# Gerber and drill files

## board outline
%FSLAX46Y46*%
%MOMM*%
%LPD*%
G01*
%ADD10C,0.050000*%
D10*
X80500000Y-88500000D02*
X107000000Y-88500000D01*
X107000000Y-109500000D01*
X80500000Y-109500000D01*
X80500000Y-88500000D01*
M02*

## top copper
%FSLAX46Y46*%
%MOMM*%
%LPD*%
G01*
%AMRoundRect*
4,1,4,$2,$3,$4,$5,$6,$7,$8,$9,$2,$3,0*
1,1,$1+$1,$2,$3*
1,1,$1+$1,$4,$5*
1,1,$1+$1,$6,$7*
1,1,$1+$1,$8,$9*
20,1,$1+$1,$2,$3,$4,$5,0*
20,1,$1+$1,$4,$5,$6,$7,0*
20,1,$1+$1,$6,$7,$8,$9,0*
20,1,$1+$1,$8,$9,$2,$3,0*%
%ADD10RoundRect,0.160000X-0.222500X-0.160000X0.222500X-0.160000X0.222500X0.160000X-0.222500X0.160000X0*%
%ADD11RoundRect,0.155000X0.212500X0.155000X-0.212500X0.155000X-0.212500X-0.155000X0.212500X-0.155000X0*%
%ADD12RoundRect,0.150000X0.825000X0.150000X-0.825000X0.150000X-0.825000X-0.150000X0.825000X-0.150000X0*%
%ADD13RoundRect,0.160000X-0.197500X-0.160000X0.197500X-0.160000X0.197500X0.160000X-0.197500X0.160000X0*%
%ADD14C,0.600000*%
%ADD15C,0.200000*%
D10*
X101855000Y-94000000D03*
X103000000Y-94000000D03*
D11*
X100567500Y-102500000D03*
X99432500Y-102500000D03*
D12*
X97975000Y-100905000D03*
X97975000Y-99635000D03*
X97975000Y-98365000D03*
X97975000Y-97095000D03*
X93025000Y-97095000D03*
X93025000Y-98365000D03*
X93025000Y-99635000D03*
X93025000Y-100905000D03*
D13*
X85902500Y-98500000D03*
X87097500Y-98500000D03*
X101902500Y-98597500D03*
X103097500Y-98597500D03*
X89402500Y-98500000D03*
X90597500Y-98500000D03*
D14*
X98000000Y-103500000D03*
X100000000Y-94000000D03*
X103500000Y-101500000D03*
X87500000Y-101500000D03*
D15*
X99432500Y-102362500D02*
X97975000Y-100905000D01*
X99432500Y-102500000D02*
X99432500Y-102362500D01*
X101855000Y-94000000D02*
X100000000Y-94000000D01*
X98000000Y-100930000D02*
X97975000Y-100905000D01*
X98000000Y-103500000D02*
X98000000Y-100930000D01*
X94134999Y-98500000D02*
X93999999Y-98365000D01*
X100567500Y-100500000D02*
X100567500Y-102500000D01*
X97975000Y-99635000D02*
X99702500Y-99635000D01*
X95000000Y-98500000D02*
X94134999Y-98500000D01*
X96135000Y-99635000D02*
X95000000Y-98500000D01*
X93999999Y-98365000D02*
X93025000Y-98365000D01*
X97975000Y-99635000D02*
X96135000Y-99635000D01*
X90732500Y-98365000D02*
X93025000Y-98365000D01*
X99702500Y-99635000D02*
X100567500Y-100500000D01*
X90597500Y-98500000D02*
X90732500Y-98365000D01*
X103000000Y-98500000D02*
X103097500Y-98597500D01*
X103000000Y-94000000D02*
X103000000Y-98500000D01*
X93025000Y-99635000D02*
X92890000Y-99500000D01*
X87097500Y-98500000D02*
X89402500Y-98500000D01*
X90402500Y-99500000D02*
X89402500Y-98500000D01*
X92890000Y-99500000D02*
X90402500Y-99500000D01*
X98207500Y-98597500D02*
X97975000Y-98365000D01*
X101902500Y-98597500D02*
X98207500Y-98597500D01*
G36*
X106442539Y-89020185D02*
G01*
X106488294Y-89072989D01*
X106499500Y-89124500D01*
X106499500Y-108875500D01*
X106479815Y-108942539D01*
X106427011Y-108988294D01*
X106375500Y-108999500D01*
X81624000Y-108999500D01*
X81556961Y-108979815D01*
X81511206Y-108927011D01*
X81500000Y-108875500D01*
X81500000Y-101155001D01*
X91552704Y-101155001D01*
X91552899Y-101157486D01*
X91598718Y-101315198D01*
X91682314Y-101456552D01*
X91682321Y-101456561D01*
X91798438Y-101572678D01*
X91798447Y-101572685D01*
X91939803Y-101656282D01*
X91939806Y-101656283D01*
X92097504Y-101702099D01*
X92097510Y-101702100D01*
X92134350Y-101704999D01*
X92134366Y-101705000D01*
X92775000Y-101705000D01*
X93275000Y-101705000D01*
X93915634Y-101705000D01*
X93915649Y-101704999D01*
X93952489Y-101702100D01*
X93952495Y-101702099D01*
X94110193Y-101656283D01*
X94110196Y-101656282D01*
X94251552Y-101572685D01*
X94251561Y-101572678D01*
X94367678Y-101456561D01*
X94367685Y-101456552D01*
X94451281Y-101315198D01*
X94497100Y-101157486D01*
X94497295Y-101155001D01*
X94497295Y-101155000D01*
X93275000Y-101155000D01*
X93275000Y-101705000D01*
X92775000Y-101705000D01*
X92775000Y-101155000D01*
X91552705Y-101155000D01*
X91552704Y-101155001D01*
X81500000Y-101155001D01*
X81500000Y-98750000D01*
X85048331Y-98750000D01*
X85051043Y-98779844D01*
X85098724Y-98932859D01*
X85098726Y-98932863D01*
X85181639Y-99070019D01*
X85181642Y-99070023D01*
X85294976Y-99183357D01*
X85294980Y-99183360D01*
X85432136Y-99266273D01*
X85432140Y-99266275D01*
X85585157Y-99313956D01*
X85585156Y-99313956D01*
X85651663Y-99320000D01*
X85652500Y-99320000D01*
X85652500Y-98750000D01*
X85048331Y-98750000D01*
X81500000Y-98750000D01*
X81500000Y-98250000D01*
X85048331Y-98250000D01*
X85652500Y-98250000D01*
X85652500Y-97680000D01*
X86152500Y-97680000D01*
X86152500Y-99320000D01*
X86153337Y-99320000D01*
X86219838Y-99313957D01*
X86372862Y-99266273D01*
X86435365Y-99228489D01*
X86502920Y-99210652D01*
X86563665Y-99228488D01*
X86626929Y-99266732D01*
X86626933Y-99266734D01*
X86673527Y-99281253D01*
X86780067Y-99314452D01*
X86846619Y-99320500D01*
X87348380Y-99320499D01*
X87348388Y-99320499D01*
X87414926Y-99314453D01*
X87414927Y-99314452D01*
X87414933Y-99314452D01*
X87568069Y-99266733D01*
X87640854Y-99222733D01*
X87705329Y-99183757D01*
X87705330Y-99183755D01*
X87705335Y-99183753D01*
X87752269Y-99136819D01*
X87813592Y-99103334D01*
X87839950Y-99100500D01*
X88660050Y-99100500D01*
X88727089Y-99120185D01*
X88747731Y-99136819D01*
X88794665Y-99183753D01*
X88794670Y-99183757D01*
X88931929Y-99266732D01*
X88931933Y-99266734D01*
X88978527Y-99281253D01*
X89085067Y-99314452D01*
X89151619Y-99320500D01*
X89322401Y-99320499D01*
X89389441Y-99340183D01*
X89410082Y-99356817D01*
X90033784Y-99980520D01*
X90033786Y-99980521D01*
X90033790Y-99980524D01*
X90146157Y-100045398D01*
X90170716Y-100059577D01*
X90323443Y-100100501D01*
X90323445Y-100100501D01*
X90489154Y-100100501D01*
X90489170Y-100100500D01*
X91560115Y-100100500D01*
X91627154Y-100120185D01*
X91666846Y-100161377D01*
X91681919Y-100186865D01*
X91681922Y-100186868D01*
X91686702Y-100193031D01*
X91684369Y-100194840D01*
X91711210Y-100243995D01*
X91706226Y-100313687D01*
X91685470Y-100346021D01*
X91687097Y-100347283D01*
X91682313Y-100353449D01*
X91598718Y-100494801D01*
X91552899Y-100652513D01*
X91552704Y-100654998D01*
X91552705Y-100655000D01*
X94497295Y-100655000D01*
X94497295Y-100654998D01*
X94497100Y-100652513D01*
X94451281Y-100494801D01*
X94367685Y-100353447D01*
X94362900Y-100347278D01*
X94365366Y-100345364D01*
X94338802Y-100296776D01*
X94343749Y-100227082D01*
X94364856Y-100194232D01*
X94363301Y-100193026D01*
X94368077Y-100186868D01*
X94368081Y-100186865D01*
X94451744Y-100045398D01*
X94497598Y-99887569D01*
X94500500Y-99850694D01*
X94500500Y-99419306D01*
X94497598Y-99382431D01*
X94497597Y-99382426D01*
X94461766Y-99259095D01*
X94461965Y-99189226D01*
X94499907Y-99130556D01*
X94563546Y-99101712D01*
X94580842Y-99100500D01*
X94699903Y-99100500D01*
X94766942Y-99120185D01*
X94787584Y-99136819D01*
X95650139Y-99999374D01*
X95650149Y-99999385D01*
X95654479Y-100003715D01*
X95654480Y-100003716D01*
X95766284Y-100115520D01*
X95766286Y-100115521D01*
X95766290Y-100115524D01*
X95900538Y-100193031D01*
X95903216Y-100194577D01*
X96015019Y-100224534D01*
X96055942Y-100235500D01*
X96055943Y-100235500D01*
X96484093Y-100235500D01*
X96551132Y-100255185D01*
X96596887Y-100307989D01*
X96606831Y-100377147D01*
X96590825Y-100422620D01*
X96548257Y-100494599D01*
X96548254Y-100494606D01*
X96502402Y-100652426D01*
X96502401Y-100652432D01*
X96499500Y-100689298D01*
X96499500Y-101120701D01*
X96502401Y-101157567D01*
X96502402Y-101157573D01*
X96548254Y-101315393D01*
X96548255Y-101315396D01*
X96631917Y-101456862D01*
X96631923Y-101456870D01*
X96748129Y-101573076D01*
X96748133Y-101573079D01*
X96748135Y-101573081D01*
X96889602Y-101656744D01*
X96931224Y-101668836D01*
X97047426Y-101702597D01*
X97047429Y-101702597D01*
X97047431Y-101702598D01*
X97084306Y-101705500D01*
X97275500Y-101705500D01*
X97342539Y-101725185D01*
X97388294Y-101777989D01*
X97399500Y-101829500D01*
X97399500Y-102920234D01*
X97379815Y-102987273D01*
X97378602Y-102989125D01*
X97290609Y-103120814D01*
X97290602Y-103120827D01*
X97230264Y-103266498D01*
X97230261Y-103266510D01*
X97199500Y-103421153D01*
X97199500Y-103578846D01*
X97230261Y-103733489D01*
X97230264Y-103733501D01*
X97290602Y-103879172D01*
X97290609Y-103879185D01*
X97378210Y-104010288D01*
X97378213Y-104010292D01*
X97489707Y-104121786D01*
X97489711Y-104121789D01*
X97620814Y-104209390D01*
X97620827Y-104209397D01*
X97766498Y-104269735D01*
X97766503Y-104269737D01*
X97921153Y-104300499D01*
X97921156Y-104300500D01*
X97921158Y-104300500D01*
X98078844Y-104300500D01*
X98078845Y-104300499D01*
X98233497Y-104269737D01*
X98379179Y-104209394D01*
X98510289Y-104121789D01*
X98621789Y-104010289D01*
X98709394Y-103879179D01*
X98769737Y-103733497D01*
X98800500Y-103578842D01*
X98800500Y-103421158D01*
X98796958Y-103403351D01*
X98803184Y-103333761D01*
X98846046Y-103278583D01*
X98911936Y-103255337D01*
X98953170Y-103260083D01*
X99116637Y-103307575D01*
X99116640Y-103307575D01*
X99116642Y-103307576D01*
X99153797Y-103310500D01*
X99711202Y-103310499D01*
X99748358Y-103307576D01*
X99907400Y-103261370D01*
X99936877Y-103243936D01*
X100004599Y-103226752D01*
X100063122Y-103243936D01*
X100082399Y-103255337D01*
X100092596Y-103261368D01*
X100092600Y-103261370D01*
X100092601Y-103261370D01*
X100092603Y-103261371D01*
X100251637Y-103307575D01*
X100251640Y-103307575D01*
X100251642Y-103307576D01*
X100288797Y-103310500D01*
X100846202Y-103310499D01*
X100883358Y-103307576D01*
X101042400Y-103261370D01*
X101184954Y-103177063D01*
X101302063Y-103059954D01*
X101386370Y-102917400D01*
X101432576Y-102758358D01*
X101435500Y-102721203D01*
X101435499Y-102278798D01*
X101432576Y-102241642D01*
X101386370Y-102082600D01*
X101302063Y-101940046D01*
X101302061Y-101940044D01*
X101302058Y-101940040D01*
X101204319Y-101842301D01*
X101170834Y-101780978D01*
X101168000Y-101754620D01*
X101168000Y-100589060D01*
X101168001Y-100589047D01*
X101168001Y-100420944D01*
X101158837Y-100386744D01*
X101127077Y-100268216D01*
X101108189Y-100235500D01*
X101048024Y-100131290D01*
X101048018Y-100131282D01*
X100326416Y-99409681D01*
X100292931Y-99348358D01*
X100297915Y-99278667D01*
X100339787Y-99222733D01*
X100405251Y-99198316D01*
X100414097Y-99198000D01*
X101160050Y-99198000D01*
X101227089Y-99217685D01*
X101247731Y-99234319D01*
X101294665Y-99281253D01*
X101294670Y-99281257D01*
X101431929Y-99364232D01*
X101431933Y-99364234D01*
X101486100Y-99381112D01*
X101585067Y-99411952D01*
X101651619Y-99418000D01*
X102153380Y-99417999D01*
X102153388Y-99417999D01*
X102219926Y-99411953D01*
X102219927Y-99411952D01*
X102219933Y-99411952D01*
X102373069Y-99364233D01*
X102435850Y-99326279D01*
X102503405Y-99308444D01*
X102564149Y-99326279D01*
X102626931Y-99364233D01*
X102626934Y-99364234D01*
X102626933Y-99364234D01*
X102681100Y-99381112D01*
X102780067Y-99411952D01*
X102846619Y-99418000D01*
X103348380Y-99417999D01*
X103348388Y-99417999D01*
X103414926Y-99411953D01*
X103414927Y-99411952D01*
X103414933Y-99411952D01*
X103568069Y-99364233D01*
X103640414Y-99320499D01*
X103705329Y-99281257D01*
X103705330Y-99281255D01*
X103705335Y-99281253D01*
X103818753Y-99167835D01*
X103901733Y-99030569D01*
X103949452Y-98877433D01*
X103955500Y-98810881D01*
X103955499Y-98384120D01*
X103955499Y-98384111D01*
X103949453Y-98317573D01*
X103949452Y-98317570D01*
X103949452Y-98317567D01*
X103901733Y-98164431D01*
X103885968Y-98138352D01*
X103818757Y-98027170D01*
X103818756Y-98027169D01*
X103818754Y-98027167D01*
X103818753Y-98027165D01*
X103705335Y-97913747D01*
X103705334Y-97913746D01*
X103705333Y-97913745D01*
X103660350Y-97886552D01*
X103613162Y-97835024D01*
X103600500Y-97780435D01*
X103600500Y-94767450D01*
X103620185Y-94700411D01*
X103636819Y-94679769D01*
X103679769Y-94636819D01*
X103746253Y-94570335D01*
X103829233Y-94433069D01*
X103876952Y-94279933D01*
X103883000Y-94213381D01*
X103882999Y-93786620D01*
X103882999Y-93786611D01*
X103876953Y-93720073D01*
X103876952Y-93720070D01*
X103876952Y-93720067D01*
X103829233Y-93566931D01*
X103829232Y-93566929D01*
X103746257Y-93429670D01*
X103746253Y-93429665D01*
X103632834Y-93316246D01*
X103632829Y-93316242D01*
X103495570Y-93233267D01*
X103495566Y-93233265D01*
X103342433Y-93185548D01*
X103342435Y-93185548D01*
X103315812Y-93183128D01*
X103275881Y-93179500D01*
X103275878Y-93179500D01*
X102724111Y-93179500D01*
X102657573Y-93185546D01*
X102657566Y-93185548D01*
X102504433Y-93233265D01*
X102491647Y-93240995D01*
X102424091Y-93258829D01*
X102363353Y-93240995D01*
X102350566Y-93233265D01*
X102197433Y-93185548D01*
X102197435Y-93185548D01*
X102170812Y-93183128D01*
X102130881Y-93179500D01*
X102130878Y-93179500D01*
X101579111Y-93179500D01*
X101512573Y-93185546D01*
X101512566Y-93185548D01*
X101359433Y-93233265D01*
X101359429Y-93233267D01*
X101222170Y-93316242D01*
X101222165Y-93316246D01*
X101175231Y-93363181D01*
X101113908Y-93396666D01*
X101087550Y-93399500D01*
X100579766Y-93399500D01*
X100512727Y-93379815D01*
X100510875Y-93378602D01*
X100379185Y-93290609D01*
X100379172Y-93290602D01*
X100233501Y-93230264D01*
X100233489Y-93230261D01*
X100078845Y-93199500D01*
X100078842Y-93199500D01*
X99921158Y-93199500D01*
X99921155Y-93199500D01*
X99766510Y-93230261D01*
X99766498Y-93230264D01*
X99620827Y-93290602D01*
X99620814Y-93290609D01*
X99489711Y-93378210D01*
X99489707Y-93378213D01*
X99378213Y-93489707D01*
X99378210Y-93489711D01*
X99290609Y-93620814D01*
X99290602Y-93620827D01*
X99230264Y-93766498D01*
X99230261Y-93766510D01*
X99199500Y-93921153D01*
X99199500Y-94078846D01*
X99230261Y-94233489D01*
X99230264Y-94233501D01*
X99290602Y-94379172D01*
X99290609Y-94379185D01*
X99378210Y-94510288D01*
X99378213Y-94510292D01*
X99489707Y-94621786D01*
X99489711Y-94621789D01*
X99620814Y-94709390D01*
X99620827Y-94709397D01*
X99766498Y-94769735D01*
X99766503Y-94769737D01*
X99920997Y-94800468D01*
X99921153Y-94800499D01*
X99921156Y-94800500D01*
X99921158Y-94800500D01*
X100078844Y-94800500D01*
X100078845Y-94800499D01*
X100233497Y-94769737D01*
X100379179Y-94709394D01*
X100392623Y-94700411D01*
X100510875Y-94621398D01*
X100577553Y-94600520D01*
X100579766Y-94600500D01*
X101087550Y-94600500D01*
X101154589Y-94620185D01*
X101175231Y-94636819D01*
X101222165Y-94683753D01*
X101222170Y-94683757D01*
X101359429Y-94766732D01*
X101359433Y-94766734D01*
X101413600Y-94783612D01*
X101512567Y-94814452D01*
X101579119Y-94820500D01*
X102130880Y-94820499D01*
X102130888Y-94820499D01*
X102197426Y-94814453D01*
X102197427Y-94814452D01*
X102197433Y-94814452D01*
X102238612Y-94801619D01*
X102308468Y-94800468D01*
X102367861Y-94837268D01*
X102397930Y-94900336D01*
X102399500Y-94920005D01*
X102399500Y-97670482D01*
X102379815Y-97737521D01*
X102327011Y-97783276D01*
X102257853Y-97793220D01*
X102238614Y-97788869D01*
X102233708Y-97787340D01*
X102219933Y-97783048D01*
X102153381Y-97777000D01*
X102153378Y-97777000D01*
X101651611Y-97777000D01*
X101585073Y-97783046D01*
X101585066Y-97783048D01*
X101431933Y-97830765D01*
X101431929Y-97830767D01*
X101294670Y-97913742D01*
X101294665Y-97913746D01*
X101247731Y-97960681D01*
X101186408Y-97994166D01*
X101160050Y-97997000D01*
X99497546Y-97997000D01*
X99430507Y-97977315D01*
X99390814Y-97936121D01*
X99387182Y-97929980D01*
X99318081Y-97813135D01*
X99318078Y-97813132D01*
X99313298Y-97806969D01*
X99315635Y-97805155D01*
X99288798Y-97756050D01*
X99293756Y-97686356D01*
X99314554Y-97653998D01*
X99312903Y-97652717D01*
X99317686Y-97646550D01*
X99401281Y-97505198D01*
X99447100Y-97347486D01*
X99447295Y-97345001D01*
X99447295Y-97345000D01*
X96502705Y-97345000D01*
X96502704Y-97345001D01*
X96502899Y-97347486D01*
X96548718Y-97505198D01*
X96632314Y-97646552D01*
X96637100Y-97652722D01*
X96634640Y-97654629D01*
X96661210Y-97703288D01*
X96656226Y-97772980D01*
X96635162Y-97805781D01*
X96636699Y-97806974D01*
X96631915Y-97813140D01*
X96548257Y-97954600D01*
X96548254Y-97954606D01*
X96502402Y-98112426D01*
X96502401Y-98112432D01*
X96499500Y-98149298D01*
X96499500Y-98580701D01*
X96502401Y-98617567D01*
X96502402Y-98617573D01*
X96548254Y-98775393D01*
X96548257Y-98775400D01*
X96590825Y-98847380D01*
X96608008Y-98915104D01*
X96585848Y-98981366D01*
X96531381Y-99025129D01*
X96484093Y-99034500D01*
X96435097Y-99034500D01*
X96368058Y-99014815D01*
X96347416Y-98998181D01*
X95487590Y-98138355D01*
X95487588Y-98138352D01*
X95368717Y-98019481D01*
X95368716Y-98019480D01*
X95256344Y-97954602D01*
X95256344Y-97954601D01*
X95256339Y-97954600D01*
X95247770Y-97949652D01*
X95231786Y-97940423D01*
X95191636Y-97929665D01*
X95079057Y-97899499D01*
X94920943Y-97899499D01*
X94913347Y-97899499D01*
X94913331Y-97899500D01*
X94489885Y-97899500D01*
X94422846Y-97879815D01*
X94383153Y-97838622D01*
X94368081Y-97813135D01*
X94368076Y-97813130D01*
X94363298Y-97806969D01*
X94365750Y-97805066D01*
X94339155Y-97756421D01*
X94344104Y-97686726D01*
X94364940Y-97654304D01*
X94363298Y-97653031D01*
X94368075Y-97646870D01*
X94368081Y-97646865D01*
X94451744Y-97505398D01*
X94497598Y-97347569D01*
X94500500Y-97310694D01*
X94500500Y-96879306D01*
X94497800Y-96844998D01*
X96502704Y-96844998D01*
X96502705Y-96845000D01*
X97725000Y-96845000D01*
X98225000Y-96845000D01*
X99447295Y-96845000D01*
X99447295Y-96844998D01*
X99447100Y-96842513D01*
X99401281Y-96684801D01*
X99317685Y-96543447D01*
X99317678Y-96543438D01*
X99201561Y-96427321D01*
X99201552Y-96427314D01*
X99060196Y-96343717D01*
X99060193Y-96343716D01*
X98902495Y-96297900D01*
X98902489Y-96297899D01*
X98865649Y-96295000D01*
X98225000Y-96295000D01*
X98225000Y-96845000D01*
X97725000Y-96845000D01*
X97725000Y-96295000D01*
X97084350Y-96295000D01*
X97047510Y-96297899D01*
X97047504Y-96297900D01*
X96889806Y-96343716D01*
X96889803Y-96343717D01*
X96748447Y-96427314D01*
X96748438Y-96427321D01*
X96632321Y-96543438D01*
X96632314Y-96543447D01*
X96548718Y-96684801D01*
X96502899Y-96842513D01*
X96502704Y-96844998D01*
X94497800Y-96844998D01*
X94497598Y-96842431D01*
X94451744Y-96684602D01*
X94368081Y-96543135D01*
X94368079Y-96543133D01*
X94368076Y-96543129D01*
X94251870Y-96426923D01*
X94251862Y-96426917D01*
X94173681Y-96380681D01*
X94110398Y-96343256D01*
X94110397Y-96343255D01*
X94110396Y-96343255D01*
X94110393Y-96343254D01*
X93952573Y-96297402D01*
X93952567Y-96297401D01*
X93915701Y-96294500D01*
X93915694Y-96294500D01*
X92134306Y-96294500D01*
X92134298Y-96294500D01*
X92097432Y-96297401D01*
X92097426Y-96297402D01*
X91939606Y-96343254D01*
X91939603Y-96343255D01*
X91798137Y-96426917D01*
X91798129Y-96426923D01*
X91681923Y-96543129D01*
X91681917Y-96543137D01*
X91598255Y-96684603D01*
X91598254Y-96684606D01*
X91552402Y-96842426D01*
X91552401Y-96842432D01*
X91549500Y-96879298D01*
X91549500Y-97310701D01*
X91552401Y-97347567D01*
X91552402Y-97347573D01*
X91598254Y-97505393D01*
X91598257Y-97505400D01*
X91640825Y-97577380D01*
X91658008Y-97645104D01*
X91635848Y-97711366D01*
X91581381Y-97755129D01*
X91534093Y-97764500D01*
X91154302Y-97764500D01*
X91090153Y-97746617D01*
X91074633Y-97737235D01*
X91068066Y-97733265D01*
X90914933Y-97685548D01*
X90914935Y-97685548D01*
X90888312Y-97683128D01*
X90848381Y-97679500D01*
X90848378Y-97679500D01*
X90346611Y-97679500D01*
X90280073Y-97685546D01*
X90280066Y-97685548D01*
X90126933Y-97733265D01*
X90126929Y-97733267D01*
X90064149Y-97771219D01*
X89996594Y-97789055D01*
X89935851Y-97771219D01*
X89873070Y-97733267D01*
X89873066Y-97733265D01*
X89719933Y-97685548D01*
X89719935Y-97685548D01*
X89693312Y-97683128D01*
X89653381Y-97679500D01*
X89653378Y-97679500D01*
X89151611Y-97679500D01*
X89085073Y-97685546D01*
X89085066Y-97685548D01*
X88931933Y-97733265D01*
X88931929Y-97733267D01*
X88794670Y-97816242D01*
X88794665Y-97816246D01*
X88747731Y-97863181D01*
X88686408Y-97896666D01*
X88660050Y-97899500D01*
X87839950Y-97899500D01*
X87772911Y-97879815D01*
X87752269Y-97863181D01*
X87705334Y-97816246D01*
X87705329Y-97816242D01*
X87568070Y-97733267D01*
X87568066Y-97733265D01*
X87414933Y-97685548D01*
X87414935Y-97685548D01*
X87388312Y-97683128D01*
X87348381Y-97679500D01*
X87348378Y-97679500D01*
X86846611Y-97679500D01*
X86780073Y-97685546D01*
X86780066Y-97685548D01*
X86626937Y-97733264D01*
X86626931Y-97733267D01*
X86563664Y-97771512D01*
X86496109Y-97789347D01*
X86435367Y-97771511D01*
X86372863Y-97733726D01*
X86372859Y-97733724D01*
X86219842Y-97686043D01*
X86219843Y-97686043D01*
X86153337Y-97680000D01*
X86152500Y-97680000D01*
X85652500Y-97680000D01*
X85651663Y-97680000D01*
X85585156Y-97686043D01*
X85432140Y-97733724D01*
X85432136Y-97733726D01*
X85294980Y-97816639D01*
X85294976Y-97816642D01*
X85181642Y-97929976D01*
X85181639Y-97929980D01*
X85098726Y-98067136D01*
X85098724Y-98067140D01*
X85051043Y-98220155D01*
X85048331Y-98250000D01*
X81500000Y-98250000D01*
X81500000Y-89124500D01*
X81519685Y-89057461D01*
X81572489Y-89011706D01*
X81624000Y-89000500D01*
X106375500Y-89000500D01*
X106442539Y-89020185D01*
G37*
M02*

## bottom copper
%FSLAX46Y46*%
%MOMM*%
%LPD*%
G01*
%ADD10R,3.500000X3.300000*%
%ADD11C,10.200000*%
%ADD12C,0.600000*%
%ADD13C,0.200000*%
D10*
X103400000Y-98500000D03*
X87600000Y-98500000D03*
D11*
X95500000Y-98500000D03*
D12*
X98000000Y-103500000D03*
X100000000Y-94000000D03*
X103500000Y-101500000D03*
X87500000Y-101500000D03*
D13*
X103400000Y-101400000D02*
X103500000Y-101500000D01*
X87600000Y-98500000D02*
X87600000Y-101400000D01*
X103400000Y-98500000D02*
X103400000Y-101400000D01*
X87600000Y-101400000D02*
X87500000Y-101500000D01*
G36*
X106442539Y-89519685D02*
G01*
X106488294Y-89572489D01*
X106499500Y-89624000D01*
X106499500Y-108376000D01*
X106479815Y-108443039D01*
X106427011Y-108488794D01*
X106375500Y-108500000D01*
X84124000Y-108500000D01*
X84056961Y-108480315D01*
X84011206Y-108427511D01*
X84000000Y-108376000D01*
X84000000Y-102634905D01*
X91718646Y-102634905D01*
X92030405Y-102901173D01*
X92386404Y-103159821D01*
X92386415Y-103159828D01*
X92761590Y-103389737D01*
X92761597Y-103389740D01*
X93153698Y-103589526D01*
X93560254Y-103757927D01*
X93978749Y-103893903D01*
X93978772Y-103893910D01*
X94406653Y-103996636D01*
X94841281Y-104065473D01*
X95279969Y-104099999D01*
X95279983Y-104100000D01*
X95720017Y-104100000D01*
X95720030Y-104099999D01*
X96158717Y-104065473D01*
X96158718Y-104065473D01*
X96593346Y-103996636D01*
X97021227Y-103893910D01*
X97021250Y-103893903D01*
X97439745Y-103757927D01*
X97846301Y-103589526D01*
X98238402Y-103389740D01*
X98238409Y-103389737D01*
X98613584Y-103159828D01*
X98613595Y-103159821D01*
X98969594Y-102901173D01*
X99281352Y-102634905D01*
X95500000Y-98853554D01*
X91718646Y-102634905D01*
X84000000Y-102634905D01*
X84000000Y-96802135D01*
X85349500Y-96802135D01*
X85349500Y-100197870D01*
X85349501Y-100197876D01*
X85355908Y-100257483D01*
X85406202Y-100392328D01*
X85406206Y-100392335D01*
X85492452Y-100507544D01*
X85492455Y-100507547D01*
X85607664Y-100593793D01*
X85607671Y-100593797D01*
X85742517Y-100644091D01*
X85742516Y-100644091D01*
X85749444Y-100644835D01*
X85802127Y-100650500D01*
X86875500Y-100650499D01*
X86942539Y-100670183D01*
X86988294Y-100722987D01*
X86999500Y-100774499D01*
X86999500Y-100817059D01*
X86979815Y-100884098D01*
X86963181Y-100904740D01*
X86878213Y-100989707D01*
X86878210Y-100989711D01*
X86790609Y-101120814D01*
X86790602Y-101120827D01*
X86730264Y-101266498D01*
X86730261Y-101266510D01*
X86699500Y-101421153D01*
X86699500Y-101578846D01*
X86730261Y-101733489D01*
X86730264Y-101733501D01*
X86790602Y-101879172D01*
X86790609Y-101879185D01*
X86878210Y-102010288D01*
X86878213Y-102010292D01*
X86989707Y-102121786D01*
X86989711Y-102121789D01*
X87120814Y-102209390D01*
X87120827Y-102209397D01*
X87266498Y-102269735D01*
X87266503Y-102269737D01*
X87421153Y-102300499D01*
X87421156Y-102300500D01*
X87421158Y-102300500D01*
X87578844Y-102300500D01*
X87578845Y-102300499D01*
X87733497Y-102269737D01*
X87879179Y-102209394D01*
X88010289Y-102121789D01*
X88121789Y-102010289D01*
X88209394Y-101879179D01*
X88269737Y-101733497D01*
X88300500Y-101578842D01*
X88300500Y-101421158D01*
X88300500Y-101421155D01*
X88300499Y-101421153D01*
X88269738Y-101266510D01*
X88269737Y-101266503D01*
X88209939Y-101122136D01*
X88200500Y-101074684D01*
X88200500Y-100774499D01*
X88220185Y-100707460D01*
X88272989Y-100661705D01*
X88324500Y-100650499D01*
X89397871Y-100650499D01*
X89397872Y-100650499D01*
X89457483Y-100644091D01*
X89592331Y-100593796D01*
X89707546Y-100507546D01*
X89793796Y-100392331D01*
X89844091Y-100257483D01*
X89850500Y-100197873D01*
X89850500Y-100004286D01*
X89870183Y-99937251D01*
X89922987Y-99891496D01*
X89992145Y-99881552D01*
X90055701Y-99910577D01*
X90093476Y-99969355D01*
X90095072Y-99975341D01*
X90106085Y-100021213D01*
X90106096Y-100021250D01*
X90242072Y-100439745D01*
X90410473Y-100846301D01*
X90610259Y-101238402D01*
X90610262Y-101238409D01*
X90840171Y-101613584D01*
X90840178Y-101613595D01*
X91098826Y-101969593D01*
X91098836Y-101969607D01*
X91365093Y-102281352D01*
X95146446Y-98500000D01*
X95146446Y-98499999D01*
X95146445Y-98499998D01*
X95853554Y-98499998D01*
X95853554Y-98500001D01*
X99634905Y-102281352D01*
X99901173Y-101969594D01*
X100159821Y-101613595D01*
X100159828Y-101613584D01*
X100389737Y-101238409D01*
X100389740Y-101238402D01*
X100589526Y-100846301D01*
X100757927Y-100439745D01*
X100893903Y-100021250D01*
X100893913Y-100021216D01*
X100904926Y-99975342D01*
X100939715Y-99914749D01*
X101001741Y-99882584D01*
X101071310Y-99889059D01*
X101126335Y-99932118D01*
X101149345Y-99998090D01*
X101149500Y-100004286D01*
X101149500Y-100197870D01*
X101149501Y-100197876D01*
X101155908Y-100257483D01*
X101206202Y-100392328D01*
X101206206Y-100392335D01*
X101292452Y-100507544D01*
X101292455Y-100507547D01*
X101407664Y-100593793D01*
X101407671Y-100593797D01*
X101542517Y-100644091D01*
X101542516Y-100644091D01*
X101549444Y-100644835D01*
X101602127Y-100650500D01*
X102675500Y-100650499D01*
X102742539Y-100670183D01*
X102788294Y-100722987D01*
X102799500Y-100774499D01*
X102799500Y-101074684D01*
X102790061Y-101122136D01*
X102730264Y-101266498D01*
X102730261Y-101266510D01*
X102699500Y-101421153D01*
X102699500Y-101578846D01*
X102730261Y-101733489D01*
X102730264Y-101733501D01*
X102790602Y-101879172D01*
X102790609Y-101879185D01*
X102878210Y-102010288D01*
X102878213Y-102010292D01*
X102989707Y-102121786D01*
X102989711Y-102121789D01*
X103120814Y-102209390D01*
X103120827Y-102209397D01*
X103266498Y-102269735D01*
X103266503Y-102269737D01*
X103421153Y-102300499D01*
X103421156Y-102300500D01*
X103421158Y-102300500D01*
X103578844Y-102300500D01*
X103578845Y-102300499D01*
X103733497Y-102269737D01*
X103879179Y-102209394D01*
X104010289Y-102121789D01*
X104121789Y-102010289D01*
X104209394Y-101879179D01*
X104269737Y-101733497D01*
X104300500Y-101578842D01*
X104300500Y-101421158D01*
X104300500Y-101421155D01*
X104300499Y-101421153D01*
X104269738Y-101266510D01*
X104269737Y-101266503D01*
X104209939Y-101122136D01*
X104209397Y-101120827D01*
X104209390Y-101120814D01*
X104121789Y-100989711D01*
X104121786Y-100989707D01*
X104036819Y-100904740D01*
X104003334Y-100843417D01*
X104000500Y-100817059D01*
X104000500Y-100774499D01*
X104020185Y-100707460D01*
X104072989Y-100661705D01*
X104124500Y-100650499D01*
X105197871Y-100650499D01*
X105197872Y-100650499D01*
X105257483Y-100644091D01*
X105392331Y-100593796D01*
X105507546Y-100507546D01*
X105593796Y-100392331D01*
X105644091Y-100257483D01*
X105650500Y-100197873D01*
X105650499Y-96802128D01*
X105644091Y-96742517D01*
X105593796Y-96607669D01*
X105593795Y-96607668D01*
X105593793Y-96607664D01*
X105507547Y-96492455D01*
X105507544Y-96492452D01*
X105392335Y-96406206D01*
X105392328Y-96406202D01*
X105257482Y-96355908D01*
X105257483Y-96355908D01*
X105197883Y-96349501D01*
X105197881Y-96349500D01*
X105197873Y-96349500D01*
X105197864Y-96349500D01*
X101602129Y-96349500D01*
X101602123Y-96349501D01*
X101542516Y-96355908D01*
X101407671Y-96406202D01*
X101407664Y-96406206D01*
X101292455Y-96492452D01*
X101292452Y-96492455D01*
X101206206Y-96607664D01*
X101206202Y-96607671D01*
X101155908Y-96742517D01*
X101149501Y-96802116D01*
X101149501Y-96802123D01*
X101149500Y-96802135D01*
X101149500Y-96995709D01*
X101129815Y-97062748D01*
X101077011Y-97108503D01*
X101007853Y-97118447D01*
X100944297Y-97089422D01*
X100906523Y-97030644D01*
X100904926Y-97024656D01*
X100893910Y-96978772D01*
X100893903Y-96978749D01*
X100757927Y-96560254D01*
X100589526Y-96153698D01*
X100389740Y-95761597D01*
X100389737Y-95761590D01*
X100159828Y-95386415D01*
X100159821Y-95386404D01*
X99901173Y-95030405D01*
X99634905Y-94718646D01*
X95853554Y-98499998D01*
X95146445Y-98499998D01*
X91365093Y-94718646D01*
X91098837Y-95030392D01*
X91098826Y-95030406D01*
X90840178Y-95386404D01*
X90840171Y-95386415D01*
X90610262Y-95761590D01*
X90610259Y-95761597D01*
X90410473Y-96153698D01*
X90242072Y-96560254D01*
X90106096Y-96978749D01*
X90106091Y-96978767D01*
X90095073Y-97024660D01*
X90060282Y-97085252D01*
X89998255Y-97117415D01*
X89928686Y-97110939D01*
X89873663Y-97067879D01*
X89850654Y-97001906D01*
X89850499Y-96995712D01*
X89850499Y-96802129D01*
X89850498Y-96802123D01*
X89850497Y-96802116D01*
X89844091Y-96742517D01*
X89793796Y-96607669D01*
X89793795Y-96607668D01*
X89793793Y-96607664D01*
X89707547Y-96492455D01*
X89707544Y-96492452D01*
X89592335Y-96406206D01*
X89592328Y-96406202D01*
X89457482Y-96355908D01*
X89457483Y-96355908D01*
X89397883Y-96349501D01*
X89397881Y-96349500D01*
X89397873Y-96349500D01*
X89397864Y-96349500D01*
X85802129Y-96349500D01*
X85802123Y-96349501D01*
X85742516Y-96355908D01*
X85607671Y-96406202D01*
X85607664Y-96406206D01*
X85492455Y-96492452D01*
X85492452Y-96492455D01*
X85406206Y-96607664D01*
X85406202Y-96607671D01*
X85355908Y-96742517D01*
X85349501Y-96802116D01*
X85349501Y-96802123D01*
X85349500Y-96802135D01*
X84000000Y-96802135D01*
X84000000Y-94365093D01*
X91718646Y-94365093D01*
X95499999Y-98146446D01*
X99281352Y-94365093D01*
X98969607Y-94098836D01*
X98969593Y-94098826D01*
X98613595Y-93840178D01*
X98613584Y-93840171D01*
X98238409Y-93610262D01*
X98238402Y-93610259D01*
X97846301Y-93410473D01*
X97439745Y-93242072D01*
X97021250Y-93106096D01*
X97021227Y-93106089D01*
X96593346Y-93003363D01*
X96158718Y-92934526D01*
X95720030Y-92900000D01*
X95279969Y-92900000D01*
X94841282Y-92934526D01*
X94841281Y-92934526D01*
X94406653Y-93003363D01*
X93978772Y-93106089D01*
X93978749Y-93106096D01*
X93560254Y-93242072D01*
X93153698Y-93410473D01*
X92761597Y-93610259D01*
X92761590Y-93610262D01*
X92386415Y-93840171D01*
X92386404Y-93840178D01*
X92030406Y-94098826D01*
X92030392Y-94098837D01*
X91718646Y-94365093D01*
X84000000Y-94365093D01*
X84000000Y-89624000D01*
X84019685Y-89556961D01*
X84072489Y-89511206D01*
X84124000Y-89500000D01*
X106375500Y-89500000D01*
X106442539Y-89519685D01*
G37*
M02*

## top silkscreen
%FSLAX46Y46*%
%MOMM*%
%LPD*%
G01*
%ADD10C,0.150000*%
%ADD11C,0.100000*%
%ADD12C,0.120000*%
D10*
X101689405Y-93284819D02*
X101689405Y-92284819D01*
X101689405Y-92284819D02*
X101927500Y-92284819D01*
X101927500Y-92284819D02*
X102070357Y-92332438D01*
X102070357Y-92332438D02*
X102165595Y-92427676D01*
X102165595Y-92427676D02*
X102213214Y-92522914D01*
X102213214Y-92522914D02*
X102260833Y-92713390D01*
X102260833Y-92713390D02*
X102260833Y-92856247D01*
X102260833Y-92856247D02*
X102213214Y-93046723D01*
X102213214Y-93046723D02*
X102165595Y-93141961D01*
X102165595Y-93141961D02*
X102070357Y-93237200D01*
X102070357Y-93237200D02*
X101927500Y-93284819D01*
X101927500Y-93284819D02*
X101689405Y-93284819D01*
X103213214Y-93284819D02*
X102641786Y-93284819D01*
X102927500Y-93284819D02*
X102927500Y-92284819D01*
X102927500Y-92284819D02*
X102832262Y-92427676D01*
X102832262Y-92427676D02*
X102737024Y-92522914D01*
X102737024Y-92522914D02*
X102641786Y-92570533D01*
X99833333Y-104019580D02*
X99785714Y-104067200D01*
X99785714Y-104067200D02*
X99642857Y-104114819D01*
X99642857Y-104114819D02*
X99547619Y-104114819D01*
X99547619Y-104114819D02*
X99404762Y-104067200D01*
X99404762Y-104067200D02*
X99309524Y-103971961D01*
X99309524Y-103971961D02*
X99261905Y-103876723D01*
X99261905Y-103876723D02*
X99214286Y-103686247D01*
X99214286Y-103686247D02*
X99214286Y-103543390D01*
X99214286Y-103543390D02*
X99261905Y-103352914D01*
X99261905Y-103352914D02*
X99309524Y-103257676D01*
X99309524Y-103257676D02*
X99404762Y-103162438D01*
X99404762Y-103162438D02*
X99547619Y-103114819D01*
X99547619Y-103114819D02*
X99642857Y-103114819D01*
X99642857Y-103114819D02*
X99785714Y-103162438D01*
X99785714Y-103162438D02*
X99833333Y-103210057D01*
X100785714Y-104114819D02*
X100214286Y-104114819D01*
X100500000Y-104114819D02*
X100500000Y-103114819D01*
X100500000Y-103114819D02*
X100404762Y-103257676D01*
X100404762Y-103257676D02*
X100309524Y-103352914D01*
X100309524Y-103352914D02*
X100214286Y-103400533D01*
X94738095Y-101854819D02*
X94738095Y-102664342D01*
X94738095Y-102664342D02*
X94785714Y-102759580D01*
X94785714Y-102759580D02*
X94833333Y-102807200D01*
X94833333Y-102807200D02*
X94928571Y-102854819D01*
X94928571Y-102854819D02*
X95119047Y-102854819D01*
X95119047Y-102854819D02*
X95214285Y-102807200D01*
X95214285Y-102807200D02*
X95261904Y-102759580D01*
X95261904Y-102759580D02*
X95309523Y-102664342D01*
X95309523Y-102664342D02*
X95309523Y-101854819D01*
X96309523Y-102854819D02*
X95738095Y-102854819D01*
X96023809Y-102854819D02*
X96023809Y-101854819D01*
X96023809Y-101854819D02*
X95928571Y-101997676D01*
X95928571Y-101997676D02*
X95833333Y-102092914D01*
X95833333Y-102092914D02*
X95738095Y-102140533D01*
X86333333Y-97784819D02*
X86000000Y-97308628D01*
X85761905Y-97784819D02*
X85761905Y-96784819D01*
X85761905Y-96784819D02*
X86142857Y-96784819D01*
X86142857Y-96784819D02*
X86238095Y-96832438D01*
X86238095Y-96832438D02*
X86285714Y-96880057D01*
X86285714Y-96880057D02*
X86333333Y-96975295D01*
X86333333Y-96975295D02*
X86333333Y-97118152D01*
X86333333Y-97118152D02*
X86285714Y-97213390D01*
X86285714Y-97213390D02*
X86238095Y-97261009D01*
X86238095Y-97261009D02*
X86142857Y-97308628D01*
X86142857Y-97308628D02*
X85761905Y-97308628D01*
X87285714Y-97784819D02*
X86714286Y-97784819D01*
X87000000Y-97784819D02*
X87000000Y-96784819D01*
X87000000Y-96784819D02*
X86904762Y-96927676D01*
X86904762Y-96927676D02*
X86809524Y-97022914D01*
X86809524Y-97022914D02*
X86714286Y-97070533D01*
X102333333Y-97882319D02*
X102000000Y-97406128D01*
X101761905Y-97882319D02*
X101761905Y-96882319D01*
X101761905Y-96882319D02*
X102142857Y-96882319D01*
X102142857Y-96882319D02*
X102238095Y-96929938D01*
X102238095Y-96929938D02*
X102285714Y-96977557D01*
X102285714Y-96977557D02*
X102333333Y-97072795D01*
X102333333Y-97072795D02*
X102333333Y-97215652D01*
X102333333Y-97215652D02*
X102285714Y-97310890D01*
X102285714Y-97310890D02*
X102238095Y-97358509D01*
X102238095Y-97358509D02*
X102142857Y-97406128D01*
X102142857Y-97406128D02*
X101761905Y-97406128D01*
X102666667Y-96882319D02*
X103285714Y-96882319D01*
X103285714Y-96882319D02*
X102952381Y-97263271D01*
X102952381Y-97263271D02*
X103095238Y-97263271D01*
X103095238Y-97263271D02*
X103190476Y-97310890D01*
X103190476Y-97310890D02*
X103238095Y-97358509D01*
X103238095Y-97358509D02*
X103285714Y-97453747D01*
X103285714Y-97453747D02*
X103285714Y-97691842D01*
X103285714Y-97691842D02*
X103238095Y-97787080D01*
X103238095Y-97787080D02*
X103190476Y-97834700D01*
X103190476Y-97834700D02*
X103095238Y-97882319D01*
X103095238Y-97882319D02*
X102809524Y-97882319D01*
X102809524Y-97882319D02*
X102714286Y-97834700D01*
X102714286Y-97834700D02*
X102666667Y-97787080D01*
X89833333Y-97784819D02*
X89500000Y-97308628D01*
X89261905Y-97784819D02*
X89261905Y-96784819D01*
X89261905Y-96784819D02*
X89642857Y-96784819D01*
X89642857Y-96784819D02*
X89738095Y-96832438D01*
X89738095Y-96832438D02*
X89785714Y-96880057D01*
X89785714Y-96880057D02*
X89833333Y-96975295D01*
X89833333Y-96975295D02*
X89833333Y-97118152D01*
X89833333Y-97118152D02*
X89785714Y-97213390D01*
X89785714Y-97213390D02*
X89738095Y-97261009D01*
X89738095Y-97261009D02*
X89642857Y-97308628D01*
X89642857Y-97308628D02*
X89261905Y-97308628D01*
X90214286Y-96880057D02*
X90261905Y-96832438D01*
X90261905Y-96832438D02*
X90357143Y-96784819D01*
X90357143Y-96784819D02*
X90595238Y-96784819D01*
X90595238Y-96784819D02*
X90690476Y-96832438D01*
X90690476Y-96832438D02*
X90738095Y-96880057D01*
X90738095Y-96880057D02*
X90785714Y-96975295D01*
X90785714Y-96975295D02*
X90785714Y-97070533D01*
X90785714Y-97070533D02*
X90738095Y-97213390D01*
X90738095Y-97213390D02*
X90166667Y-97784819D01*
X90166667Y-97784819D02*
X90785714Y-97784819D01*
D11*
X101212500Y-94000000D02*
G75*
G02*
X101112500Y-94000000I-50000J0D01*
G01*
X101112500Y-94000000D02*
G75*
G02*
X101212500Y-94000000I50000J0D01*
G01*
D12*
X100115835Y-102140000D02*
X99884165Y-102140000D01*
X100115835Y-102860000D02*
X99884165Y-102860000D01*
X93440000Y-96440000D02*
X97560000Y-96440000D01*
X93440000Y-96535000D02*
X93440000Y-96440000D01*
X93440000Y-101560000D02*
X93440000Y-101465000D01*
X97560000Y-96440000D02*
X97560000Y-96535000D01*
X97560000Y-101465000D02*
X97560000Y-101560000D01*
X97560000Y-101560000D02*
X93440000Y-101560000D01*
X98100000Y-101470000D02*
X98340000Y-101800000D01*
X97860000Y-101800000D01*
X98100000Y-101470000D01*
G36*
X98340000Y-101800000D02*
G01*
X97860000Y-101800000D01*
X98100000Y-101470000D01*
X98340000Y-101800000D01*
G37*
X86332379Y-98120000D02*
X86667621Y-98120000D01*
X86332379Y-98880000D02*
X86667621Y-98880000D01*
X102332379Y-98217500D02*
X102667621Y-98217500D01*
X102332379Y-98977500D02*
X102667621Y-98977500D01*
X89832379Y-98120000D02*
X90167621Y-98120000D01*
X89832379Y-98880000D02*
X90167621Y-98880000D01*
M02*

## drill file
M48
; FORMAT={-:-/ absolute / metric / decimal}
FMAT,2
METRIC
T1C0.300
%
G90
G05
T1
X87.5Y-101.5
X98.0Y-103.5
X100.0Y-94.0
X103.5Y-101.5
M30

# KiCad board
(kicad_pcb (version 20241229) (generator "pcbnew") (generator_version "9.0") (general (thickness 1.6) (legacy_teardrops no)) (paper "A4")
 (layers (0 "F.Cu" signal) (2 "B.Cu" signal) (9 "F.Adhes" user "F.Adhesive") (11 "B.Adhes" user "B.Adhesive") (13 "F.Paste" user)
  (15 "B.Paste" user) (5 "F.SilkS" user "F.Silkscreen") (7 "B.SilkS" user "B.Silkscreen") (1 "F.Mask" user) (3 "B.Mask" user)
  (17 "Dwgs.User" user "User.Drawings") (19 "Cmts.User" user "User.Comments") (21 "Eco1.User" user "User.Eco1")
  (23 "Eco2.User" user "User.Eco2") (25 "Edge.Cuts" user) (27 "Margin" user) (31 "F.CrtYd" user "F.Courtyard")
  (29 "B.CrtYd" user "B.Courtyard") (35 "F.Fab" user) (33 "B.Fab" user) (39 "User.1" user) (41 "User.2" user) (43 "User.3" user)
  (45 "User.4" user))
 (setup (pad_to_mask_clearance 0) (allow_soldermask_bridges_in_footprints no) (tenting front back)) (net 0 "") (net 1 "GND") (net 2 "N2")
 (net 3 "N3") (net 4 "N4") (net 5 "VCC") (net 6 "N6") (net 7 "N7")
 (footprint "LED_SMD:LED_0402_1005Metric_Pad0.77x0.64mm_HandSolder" (layer "F.Cu") (at 102.4275 94)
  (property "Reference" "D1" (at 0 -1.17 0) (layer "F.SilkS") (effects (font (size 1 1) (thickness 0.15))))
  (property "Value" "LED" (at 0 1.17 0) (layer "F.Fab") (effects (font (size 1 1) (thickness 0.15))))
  (fp_circle (center -1.265 0) (end -1.215 0) (stroke (width 0.1) (type solid)) (fill no) (layer "F.SilkS"))
  (pad "1" smd roundrect (at -0.5725 0) (size 0.765 0.64) (layers "F.Cu" "F.Mask" "F.Paste") (roundrect_rratio 0.25) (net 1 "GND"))
  (pad "2" smd roundrect (at 0.5725 0) (size 0.765 0.64) (layers "F.Cu" "F.Mask" "F.Paste") (roundrect_rratio 0.25) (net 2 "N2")))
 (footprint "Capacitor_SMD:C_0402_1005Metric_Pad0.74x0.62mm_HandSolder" (layer "F.Cu") (at 100 102.5 180)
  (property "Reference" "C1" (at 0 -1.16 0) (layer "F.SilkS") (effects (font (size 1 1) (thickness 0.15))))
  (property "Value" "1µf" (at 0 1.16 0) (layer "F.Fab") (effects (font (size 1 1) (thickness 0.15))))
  (fp_line (start -0.115835 0.36) (end 0.115835 0.36) (stroke (width 0.12) (type solid)) (layer "F.SilkS"))
  (fp_line (start -0.115835 -0.36) (end 0.115835 -0.36) (stroke (width 0.12) (type solid)) (layer "F.SilkS"))
  (pad "1" smd roundrect (at -0.5675 0 180) (size 0.735 0.62) (layers "F.Cu" "F.Mask" "F.Paste") (roundrect_rratio 0.25) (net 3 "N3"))
  (pad "2" smd roundrect (at 0.5675 0 180) (size 0.735 0.62) (layers "F.Cu" "F.Mask" "F.Paste") (roundrect_rratio 0.25) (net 1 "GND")))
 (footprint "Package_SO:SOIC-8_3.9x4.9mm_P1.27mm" (layer "F.Cu") (at 95.5 99 180)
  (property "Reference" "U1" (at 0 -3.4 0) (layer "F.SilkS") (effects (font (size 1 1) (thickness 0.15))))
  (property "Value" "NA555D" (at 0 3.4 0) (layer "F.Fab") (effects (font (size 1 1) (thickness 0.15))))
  (fp_line (start 2.06 2.56) (end -2.06 2.56) (stroke (width 0.12) (type solid)) (layer "F.SilkS"))
  (fp_line (start 2.06 2.465) (end 2.06 2.56) (stroke (width 0.12) (type solid)) (layer "F.SilkS"))
  (fp_line (start 2.06 -2.56) (end 2.06 -2.465) (stroke (width 0.12) (type solid)) (layer "F.SilkS"))
  (fp_line (start -2.06 2.56) (end -2.06 2.465) (stroke (width 0.12) (type solid)) (layer "F.SilkS"))
  (fp_line (start -2.06 -2.465) (end -2.06 -2.56) (stroke (width 0.12) (type solid)) (layer "F.SilkS"))
  (fp_line (start -2.06 -2.56) (end 2.06 -2.56) (stroke (width 0.12) (type solid)) (layer "F.SilkS"))
  (fp_poly (pts (xy -2.6 -2.47) (xy -2.84 -2.8) (xy -2.36 -2.8)) (stroke (width 0.12) (type solid)) (fill yes) (layer "F.SilkS"))
  (pad "1" smd roundrect (at -2.475 -1.905 180) (size 1.95 0.6) (layers "F.Cu" "F.Mask" "F.Paste") (roundrect_rratio 0.25) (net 1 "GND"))
  (pad "2" smd roundrect (at -2.475 -0.635 180) (size 1.95 0.6) (layers "F.Cu" "F.Mask" "F.Paste") (roundrect_rratio 0.25) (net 3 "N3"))
  (pad "3" smd roundrect (at -2.475 0.635 180) (size 1.95 0.6) (layers "F.Cu" "F.Mask" "F.Paste") (roundrect_rratio 0.25) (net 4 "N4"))
  (pad "4" smd roundrect (at -2.475 1.905 180) (size 1.95 0.6) (layers "F.Cu" "F.Mask" "F.Paste") (roundrect_rratio 0.25) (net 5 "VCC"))
  (pad "5" smd roundrect (at 2.475 1.905 180) (size 1.95 0.6) (layers "F.Cu" "F.Mask" "F.Paste") (roundrect_rratio 0.25) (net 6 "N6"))
  (pad "6" smd roundrect (at 2.475 0.635 180) (size 1.95 0.6) (layers "F.Cu" "F.Mask" "F.Paste") (roundrect_rratio 0.25) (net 3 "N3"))
  (pad "7" smd roundrect (at 2.475 -0.635 180) (size 1.95 0.6) (layers "F.Cu" "F.Mask" "F.Paste") (roundrect_rratio 0.25) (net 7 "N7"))
  (pad "8" smd roundrect (at 2.475 -1.905 180) (size 1.95 0.6) (layers "F.Cu" "F.Mask" "F.Paste") (roundrect_rratio 0.25) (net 5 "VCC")))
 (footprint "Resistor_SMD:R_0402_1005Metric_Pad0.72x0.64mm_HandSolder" (layer "F.Cu") (at 86.5 98.5)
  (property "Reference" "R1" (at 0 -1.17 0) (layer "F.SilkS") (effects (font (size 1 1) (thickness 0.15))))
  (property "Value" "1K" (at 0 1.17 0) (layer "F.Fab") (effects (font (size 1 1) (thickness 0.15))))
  (fp_line (start -0.167621 -0.38) (end 0.167621 -0.38) (stroke (width 0.12) (type solid)) (layer "F.SilkS"))
  (fp_line (start -0.167621 0.38) (end 0.167621 0.38) (stroke (width 0.12) (type solid)) (layer "F.SilkS"))
  (pad "1" smd roundrect (at -0.5975 0) (size 0.715 0.64) (layers "F.Cu" "F.Mask" "F.Paste") (roundrect_rratio 0.25) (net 5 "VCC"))
  (pad "2" smd roundrect (at 0.5975 0) (size 0.715 0.64) (layers "F.Cu" "F.Mask" "F.Paste") (roundrect_rratio 0.25) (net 7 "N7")))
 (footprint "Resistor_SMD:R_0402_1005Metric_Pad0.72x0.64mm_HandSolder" (layer "F.Cu") (at 102.5 98.5975)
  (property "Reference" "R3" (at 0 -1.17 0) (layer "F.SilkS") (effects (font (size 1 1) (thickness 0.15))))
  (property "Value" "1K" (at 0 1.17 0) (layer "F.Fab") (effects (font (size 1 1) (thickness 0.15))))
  (fp_line (start -0.167621 -0.38) (end 0.167621 -0.38) (stroke (width 0.12) (type solid)) (layer "F.SilkS"))
  (fp_line (start -0.167621 0.38) (end 0.167621 0.38) (stroke (width 0.12) (type solid)) (layer "F.SilkS"))
  (pad "1" smd roundrect (at -0.5975 0) (size 0.715 0.64) (layers "F.Cu" "F.Mask" "F.Paste") (roundrect_rratio 0.25) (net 4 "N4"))
  (pad "2" smd roundrect (at 0.5975 0) (size 0.715 0.64) (layers "F.Cu" "F.Mask" "F.Paste") (roundrect_rratio 0.25) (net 2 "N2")))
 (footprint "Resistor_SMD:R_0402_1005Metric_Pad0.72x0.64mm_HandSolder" (layer "F.Cu") (at 90 98.5)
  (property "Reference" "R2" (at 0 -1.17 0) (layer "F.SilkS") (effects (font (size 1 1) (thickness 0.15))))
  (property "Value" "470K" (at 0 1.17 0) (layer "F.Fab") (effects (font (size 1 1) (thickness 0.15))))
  (fp_line (start -0.167621 -0.38) (end 0.167621 -0.38) (stroke (width 0.12) (type solid)) (layer "F.SilkS"))
  (fp_line (start -0.167621 0.38) (end 0.167621 0.38) (stroke (width 0.12) (type solid)) (layer "F.SilkS"))
  (pad "1" smd roundrect (at -0.5975 0) (size 0.715 0.64) (layers "F.Cu" "F.Mask" "F.Paste") (roundrect_rratio 0.25) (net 7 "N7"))
  (pad "2" smd roundrect (at 0.5975 0) (size 0.715 0.64) (layers "F.Cu" "F.Mask" "F.Paste") (roundrect_rratio 0.25) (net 3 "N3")))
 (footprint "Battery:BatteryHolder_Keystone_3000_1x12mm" (layer "B.Cu") (at 95.5 98.5 180)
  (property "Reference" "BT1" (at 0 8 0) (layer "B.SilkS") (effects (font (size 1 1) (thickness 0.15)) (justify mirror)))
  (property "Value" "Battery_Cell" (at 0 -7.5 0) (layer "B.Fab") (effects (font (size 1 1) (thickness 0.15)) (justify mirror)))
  (pad "1" smd rect (at -7.9 0 180) (size 3.5 3.3) (layers "B.Cu" "B.Mask" "B.Paste") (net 5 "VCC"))
  (pad "1" smd rect (at 7.9 0 180) (size 3.5 3.3) (layers "B.Cu" "B.Mask" "B.Paste") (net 5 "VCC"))
  (pad "2" smd circle (at 0 0 180) (size 10.2 10.2) (layers "B.Cu" "B.Mask") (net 1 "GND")))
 (gr_rect (start 80.5 88.5) (end 107 109.5) (stroke (width 0.05) (type default)) (fill no) (layer "Edge.Cuts"))
 (segment (start 99.4325 102.3625) (end 97.975 100.905) (width 0.2) (layer "F.Cu") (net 1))
 (segment (start 99.4325 102.5) (end 99.4325 102.3625) (width 0.2) (layer "F.Cu") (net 1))
 (segment (start 101.855 94) (end 100 94) (width 0.2) (layer "F.Cu") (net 1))
 (segment (start 98 100.93) (end 97.975 100.905) (width 0.2) (layer "F.Cu") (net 1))
 (segment (start 98 103.5) (end 98 100.93) (width 0.2) (layer "F.Cu") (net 1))
 (via (at 98 103.5) (size 0.6) (drill 0.3) (layers "F.Cu" "B.Cu") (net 1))
 (via (at 100 94) (size 0.6) (drill 0.3) (layers "F.Cu" "B.Cu") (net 1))
 (via (at 103.5 101.5) (size 0.6) (drill 0.3) (layers "F.Cu" "B.Cu") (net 5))
 (via (at 87.5 101.5) (size 0.6) (drill 0.3) (layers "F.Cu" "B.Cu") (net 5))
 (segment (start 103.4 101.4) (end 103.5 101.5) (width 0.2) (layer "B.Cu") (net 5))
 (segment (start 87.6 98.5) (end 87.6 101.4) (width 0.2) (layer "B.Cu") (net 5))
 (segment (start 103.4 98.5) (end 103.4 101.4) (width 0.2) (layer "B.Cu") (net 5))
 (segment (start 87.6 101.4) (end 87.5 101.5) (width 0.2) (layer "B.Cu") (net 5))
 (segment (start 94.134999 98.5) (end 93.999999 98.365) (width 0.2) (layer "F.Cu") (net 3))
 (segment (start 100.5675 100.5) (end 100.5675 102.5) (width 0.2) (layer "F.Cu") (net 3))
 (segment (start 97.975 99.635) (end 99.7025 99.635) (width 0.2) (layer "F.Cu") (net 3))
 (segment (start 95 98.5) (end 94.134999 98.5) (width 0.2) (layer "F.Cu") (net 3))
 (segment (start 96.135 99.635) (end 95 98.5) (width 0.2) (layer "F.Cu") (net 3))
 (segment (start 93.999999 98.365) (end 93.025 98.365) (width 0.2) (layer "F.Cu") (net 3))
 (segment (start 97.975 99.635) (end 96.135 99.635) (width 0.2) (layer "F.Cu") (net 3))
 (segment (start 90.7325 98.365) (end 93.025 98.365) (width 0.2) (layer "F.Cu") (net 3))
 (segment (start 99.7025 99.635) (end 100.5675 100.5) (width 0.2) (layer "F.Cu") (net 3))
 (segment (start 90.5975 98.5) (end 90.7325 98.365) (width 0.2) (layer "F.Cu") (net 3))
 (segment (start 103 98.5) (end 103.0975 98.5975) (width 0.2) (layer "F.Cu") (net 2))
 (segment (start 103 94) (end 103 98.5) (width 0.2) (layer "F.Cu") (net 2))
 (segment (start 93.025 99.635) (end 92.89 99.5) (width 0.2) (layer "F.Cu") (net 7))
 (segment (start 87.0975 98.5) (end 89.4025 98.5) (width 0.2) (layer "F.Cu") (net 7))
 (segment (start 90.4025 99.5) (end 89.4025 98.5) (width 0.2) (layer "F.Cu") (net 7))
 (segment (start 92.89 99.5) (end 90.4025 99.5) (width 0.2) (layer "F.Cu") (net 7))
 (segment (start 98.2075 98.5975) (end 97.975 98.365) (width 0.2) (layer "F.Cu") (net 4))
 (segment (start 101.9025 98.5975) (end 98.2075 98.5975) (width 0.2) (layer "F.Cu") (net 4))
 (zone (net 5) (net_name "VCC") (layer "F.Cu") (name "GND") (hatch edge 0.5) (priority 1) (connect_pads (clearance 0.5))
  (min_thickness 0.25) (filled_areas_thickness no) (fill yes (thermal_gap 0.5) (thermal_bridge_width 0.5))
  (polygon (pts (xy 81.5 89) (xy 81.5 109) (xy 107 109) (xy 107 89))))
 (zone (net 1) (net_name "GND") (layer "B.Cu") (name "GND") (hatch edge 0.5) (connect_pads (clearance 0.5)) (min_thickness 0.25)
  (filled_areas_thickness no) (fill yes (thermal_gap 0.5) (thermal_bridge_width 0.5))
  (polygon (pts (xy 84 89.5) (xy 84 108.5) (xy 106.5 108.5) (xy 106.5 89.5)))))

